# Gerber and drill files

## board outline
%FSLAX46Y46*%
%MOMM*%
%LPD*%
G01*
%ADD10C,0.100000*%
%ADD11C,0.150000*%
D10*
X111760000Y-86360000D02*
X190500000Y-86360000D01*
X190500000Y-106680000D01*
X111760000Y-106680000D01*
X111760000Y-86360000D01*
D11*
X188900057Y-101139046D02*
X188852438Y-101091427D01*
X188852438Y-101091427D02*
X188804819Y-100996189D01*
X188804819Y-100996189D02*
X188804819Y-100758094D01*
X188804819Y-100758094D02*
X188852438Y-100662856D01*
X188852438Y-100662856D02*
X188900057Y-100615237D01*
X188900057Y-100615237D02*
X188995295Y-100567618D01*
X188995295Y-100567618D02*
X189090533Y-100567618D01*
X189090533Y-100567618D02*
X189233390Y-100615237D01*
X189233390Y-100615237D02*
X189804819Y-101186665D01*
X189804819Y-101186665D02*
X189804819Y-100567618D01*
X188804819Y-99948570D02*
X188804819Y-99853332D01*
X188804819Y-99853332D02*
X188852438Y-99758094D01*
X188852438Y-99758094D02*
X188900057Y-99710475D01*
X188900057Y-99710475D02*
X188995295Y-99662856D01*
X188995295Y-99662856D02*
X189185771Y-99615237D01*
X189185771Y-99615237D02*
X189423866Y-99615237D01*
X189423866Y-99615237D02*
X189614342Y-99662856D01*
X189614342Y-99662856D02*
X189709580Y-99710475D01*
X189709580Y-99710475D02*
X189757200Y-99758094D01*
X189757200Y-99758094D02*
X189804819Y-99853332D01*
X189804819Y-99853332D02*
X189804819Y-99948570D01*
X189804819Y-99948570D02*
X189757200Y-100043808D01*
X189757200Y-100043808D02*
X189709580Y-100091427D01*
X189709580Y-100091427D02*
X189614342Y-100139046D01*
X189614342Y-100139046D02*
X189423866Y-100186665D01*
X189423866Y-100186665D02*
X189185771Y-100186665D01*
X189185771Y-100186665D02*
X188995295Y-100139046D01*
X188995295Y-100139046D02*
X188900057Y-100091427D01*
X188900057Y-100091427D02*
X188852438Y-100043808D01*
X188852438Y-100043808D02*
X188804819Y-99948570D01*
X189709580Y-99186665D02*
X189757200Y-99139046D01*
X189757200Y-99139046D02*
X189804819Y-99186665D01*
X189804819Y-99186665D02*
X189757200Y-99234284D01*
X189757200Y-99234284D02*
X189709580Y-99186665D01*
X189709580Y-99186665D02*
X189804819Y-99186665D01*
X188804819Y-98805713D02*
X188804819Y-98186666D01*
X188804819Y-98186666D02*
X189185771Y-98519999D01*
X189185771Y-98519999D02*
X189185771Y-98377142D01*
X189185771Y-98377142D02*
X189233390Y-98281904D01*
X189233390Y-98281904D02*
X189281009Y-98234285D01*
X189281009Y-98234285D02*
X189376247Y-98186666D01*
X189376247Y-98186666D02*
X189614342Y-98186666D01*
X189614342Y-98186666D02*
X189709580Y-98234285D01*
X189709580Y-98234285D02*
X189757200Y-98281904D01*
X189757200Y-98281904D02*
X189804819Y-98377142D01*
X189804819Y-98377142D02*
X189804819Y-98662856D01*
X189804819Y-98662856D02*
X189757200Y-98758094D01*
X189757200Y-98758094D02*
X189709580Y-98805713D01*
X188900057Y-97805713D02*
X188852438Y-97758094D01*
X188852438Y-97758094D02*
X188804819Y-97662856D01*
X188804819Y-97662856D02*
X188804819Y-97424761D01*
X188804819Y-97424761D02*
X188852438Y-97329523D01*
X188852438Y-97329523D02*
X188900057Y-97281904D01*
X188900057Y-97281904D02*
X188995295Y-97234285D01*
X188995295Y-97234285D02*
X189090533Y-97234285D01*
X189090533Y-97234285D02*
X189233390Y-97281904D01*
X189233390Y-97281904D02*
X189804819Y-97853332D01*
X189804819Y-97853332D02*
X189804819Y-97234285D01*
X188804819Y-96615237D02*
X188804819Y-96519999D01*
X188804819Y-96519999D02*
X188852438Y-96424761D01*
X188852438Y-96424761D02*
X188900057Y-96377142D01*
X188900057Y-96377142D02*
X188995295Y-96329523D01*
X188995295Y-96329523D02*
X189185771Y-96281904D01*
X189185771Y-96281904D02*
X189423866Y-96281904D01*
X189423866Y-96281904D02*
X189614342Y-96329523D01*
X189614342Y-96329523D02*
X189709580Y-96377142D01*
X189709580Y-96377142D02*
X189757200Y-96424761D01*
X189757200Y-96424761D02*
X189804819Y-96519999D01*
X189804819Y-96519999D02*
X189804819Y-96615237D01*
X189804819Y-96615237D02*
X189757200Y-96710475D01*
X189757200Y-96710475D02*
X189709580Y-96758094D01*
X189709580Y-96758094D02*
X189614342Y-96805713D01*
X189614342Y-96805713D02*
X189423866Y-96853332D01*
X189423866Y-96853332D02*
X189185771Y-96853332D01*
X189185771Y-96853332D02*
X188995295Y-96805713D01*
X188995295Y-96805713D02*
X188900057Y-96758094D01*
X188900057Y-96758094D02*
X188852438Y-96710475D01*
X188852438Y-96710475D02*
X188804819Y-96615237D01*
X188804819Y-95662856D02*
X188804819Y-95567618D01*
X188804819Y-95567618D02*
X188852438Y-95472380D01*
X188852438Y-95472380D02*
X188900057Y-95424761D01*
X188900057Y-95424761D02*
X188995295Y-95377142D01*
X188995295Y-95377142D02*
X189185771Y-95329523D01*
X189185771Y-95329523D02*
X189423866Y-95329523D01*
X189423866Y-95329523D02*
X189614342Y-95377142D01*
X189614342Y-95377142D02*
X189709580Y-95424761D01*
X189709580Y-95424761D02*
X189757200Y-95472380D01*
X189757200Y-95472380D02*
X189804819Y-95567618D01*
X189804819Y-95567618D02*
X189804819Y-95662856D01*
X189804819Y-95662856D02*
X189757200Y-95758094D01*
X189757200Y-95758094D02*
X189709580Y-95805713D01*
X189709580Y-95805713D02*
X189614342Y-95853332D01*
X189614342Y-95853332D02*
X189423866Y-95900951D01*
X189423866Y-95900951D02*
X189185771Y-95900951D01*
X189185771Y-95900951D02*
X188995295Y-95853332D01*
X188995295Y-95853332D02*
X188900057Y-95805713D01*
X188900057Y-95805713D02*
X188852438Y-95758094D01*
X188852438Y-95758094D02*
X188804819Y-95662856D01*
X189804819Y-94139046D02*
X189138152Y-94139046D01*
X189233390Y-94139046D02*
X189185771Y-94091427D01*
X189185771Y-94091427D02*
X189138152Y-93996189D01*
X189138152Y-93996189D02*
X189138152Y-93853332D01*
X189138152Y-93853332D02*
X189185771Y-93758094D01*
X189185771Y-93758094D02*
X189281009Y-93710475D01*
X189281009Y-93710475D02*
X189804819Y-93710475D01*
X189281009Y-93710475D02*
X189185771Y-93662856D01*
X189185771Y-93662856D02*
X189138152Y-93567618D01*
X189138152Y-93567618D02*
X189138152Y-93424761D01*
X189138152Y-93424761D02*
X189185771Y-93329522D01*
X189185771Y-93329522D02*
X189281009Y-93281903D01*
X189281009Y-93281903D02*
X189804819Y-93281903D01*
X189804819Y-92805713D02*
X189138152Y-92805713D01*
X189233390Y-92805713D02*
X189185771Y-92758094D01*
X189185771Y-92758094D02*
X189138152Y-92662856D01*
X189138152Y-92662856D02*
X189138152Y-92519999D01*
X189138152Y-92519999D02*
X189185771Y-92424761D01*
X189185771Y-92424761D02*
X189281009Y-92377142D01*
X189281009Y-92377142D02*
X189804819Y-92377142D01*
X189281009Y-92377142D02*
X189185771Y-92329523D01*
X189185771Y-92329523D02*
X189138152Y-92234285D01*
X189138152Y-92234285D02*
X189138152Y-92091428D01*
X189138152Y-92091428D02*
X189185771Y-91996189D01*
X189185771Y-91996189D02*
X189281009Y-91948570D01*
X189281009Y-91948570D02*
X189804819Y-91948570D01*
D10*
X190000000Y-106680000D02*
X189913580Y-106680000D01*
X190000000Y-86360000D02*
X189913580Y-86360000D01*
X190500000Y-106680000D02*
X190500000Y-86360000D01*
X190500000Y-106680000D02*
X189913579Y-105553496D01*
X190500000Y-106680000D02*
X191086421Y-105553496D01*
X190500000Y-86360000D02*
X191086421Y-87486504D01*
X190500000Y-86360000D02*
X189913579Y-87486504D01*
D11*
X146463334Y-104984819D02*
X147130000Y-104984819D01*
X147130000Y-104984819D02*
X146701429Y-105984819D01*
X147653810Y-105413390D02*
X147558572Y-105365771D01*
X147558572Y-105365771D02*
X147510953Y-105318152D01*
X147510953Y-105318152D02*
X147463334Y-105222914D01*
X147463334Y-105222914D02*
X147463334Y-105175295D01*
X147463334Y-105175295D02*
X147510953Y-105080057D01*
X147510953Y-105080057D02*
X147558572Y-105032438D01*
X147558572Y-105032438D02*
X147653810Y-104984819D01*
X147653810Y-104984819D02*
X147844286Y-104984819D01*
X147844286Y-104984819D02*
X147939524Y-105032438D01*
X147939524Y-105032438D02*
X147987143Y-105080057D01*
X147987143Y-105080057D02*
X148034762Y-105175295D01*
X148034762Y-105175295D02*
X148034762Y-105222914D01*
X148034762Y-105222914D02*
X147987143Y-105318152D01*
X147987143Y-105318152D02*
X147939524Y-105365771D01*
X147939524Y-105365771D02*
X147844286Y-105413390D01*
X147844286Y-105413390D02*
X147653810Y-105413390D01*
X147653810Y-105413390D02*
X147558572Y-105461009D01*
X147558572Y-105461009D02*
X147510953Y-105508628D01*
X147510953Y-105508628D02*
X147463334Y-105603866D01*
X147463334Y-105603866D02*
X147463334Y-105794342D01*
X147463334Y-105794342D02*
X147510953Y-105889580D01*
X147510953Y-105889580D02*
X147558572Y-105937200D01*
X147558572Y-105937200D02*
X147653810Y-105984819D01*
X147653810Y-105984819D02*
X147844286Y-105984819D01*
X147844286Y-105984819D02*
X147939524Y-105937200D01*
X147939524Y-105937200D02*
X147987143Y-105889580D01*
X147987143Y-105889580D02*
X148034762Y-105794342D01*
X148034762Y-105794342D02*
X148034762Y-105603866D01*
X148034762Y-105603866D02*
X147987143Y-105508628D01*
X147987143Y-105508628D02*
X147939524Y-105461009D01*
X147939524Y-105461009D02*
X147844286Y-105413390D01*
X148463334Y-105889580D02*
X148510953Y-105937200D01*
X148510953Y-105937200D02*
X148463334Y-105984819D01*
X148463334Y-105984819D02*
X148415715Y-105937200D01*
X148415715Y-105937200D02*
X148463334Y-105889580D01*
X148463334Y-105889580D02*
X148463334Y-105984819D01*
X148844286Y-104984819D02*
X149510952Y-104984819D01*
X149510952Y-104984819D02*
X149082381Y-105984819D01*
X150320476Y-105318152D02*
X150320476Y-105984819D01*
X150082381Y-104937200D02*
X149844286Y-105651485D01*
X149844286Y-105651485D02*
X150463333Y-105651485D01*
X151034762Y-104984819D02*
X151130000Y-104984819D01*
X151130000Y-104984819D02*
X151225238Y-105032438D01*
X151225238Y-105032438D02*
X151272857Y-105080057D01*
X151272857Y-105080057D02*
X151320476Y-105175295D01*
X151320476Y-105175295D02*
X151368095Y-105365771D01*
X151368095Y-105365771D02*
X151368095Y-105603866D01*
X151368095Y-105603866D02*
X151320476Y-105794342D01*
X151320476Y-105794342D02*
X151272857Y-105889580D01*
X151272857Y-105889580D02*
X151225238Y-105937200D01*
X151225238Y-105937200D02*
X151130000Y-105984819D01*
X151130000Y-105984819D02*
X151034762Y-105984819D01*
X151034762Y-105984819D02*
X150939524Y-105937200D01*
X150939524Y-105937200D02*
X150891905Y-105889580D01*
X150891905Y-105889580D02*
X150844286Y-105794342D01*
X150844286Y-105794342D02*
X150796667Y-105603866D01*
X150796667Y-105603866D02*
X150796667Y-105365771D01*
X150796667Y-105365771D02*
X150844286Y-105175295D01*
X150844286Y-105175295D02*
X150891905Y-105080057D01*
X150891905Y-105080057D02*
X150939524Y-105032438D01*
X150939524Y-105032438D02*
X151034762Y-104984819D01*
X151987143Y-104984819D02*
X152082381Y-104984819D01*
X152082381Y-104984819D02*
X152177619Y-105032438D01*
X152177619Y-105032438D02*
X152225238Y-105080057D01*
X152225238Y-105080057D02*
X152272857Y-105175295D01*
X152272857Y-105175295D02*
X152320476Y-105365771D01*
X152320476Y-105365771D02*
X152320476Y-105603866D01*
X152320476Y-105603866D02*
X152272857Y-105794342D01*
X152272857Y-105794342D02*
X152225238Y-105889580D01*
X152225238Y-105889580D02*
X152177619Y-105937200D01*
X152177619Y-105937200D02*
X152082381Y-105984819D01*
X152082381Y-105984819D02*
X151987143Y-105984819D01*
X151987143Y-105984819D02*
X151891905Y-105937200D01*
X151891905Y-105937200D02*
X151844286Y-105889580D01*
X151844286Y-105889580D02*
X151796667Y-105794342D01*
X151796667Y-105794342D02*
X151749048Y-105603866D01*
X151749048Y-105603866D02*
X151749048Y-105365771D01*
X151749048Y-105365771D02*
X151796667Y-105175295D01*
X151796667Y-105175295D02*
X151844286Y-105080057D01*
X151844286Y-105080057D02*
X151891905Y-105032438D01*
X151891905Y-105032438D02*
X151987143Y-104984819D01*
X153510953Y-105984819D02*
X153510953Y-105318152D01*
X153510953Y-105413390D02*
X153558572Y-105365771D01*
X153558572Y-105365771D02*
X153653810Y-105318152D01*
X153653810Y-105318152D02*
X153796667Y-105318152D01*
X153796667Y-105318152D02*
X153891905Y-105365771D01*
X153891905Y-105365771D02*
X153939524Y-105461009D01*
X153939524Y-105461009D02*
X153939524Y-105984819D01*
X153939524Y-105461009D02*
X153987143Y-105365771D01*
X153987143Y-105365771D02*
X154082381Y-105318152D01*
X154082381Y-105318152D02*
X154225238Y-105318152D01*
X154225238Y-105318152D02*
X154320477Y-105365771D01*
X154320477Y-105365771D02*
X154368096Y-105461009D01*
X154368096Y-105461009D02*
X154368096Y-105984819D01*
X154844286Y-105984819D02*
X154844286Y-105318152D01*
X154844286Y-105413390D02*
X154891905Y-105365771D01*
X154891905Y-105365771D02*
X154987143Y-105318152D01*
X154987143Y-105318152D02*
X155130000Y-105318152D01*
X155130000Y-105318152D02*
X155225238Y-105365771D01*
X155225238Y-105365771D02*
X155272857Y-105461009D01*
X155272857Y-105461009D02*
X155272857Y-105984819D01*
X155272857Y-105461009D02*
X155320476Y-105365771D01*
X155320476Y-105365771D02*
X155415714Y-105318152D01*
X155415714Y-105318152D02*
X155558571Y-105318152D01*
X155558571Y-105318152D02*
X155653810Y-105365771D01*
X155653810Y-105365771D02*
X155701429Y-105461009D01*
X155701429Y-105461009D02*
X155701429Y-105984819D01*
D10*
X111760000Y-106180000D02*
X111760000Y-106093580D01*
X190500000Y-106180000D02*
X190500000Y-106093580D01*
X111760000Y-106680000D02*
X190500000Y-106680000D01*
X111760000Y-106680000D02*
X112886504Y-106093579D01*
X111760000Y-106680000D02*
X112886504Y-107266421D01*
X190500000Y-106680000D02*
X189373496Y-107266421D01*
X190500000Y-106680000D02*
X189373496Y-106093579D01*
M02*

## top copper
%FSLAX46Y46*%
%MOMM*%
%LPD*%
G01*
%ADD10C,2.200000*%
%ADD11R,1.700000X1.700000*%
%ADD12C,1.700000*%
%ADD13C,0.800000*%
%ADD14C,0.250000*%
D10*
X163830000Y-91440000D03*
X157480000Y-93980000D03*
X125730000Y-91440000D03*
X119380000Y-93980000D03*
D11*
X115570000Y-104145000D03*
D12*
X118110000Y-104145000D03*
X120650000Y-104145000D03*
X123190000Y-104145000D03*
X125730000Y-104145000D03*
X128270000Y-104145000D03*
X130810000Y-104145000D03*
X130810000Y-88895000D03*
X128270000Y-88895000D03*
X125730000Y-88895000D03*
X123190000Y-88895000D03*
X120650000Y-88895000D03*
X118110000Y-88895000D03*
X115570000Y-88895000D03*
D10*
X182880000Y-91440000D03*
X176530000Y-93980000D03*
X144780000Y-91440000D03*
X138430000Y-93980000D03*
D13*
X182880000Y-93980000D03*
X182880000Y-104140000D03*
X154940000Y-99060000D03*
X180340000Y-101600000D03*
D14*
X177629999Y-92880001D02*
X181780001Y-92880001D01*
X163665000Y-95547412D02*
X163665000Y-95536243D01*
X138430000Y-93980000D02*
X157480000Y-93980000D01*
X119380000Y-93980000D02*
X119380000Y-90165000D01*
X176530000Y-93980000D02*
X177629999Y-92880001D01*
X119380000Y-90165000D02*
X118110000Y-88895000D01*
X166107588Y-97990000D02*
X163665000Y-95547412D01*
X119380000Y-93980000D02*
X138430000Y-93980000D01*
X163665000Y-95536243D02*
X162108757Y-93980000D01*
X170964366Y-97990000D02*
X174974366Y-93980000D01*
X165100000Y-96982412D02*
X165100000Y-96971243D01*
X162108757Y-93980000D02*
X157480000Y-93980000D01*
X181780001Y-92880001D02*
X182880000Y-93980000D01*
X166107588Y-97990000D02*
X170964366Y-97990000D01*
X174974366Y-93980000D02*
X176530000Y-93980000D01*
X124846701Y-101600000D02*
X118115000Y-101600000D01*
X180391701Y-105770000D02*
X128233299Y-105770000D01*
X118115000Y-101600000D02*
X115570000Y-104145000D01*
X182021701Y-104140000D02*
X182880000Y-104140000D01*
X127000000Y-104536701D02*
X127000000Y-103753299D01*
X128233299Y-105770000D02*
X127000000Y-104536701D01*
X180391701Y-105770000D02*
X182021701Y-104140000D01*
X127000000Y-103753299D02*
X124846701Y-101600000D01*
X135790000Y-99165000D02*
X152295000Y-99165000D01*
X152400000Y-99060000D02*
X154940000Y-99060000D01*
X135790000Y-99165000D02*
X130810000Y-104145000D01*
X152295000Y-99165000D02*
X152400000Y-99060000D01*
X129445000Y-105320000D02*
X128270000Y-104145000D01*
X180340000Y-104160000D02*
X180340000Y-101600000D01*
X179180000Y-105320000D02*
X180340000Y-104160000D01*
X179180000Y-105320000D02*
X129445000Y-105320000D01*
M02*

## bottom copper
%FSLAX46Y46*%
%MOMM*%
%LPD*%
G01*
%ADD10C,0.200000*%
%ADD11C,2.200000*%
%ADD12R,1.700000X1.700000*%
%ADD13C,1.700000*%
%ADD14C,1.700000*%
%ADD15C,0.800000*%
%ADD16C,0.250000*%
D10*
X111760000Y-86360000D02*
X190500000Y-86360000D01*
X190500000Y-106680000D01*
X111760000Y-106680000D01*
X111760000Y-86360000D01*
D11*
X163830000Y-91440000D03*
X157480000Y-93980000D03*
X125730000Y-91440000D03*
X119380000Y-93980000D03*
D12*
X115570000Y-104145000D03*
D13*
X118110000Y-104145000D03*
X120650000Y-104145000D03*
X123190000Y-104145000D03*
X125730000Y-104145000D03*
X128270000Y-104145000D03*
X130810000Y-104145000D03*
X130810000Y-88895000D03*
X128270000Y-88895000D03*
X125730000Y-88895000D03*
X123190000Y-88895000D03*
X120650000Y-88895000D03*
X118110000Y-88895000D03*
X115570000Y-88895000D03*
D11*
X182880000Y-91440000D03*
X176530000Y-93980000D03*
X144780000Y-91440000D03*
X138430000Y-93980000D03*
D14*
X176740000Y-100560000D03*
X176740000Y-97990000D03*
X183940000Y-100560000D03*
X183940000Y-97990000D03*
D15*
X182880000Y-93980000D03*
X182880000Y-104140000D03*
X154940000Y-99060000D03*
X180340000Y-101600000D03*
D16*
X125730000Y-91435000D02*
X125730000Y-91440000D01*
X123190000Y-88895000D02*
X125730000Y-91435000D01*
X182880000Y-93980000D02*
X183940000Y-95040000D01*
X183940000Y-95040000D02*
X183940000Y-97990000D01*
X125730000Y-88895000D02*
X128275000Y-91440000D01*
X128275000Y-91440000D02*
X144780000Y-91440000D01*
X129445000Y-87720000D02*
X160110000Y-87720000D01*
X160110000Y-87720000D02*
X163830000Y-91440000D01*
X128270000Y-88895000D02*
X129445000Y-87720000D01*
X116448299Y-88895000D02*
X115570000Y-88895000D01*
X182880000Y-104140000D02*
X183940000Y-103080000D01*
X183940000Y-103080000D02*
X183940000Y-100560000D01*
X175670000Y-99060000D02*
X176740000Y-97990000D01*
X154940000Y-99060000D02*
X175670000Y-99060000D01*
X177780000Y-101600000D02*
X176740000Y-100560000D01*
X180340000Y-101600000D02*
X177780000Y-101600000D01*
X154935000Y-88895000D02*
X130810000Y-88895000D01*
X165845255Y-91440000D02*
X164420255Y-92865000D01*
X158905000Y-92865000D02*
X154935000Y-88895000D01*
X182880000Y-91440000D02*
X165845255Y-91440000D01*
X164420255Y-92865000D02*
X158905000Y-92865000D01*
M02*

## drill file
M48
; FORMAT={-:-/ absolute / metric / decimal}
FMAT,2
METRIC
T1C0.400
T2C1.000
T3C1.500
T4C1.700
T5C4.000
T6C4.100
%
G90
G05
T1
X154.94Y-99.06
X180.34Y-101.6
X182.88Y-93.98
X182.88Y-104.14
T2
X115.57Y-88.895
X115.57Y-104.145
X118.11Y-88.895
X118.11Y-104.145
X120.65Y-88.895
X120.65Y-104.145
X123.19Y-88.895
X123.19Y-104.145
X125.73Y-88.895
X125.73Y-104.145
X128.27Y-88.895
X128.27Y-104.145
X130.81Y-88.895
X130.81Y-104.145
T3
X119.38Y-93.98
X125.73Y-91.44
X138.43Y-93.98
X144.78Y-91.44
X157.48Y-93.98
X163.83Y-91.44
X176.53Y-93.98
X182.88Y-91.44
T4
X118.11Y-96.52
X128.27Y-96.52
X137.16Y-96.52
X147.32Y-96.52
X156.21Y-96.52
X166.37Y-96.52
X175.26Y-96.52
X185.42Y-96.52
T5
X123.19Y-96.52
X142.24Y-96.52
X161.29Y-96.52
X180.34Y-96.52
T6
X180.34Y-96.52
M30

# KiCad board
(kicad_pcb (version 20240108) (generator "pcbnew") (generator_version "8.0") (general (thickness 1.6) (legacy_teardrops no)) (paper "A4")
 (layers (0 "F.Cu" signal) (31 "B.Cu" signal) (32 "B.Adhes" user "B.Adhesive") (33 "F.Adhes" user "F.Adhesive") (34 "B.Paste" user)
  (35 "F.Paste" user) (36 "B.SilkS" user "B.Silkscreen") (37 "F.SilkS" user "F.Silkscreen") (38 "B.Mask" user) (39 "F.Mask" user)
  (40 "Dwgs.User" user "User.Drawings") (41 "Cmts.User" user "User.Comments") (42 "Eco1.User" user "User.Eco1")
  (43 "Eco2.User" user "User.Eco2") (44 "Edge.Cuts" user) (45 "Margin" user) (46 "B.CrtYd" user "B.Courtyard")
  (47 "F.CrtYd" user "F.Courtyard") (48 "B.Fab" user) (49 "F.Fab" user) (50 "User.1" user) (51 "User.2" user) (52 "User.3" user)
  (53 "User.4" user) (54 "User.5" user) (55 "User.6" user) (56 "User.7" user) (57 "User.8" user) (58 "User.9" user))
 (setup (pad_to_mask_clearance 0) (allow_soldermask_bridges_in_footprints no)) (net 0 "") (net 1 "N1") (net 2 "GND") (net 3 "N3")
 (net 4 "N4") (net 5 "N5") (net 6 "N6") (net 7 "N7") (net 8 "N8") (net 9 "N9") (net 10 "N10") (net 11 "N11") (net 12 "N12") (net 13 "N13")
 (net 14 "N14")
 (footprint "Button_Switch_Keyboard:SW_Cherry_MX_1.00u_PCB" (layer "F.Cu") (at 163.83 91.44)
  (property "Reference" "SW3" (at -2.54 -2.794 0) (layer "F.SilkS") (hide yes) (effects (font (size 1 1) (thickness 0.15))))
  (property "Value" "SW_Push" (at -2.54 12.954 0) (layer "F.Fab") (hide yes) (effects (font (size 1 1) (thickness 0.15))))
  (pad "" np_thru_hole circle (at -7.62 5.08) (size 1.7 1.7) (drill 1.7) (layers "*.Cu" "*.Mask"))
  (pad "" np_thru_hole circle (at -2.54 5.08) (size 4 4) (drill 4) (layers "*.Cu" "*.Mask"))
  (pad "" np_thru_hole circle (at 2.54 5.08) (size 1.7 1.7) (drill 1.7) (layers "*.Cu" "*.Mask"))
  (pad "1" thru_hole circle (at 0 0) (size 2.2 2.2) (drill 1.5) (layers "*.Cu" "*.Mask") (remove_unused_layers no) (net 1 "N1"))
  (pad "2" thru_hole circle (at -6.35 2.54) (size 2.2 2.2) (drill 1.5) (layers "*.Cu" "*.Mask") (remove_unused_layers no) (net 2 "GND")))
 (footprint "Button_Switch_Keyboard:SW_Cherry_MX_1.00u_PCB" (layer "F.Cu") (at 125.73 91.44)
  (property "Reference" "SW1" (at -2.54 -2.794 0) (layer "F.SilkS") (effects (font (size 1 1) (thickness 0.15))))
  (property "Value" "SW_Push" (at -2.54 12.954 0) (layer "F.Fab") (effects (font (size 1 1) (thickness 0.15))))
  (pad "" np_thru_hole circle (at -7.62 5.08) (size 1.7 1.7) (drill 1.7) (layers "*.Cu" "*.Mask"))
  (pad "" np_thru_hole circle (at -2.54 5.08) (size 4 4) (drill 4) (layers "*.Cu" "*.Mask"))
  (pad "" np_thru_hole circle (at 2.54 5.08) (size 1.7 1.7) (drill 1.7) (layers "*.Cu" "*.Mask"))
  (pad "1" thru_hole circle (at 0 0) (size 2.2 2.2) (drill 1.5) (layers "*.Cu" "*.Mask") (remove_unused_layers no) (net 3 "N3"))
  (pad "2" thru_hole circle (at -6.35 2.54) (size 2.2 2.2) (drill 1.5) (layers "*.Cu" "*.Mask") (remove_unused_layers no) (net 2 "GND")))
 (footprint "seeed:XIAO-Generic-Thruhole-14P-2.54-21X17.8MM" (layer "F.Cu") (at 123.19 96.52 90)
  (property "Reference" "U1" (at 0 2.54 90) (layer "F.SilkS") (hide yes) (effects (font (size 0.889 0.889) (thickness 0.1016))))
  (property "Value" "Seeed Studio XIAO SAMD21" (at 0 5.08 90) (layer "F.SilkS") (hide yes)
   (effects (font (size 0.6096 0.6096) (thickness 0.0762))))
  (pad "1" thru_hole rect (at -7.625 -7.62 90) (size 1.7 1.7) (drill 1) (layers "*.Cu" "*.Mask") (remove_unused_layers no) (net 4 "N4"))
  (pad "2" thru_hole circle (at -7.625 -5.08 90) (size 1.7 1.7) (drill 1) (layers "*.Cu" "*.Mask") (remove_unused_layers no) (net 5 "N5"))
  (pad "3" thru_hole circle (at -7.625 -2.54 90) (size 1.7 1.7) (drill 1) (layers "*.Cu" "*.Mask") (remove_unused_layers no) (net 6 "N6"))
  (pad "4" thru_hole circle (at -7.625 0 90) (size 1.7 1.7) (drill 1) (layers "*.Cu" "*.Mask") (remove_unused_layers no) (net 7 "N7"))
  (pad "5" thru_hole circle (at -7.625 2.54 90) (size 1.7 1.7) (drill 1) (layers "*.Cu" "*.Mask") (remove_unused_layers no) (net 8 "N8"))
  (pad "6" thru_hole circle (at -7.625 5.08 270) (size 1.7 1.7) (drill 1) (layers "*.Cu" "*.Mask") (remove_unused_layers no) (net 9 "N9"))
  (pad "7" thru_hole circle (at -7.625 7.62 90) (size 1.7 1.7) (drill 1) (layers "*.Cu" "*.Mask") (remove_unused_layers no) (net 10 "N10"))
  (pad "8" thru_hole circle (at 7.625 7.62 90) (size 1.7 1.7) (drill 1) (layers "*.Cu" "*.Mask") (remove_unused_layers no) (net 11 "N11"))
  (pad "9" thru_hole circle (at 7.625 5.08 90) (size 1.7 1.7) (drill 1) (layers "*.Cu" "*.Mask") (remove_unused_layers no) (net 1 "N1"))
  (pad "10" thru_hole circle (at 7.625 2.54 90) (size 1.7 1.7) (drill 1) (layers "*.Cu" "*.Mask") (remove_unused_layers no) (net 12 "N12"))
  (pad "11" thru_hole circle (at 7.625 0 90) (size 1.7 1.7) (drill 1) (layers "*.Cu" "*.Mask") (remove_unused_layers no) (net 3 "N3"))
  (pad "12" thru_hole circle (at 7.625 -2.54 90) (size 1.7 1.7) (drill 1) (layers "*.Cu" "*.Mask") (remove_unused_layers no) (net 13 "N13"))
  (pad "13" thru_hole circle (at 7.625 -5.08 90) (size 1.7 1.7) (drill 1) (layers "*.Cu" "*.Mask") (remove_unused_layers no) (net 2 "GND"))
  (pad "14" thru_hole circle (at 7.625 -7.62 90) (size 1.7 1.7) (drill 1) (layers "*.Cu" "*.Mask") (remove_unused_layers no) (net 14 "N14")))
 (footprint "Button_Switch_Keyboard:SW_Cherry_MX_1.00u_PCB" (layer "F.Cu") (at 182.88 91.44)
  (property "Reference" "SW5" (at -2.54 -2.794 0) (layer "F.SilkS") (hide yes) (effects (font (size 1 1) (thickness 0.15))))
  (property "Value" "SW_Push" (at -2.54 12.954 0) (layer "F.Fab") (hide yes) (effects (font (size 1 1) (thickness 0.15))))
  (pad "" np_thru_hole circle (at -7.62 5.08) (size 1.7 1.7) (drill 1.7) (layers "*.Cu" "*.Mask"))
  (pad "" np_thru_hole circle (at -2.54 5.08) (size 4 4) (drill 4) (layers "*.Cu" "*.Mask"))
  (pad "" np_thru_hole circle (at 2.54 5.08) (size 1.7 1.7) (drill 1.7) (layers "*.Cu" "*.Mask"))
  (pad "1" thru_hole circle (at 0 0) (size 2.2 2.2) (drill 1.5) (layers "*.Cu" "*.Mask") (remove_unused_layers no) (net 11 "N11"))
  (pad "2" thru_hole circle (at -6.35 2.54) (size 2.2 2.2) (drill 1.5) (layers "*.Cu" "*.Mask") (remove_unused_layers no) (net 2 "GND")))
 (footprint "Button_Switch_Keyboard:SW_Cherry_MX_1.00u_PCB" (layer "F.Cu") (at 144.78 91.44)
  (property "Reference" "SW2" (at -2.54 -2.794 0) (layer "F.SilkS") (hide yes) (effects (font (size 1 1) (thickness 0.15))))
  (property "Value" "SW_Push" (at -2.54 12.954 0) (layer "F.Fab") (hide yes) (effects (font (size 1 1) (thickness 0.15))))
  (pad "" np_thru_hole circle (at -7.62 5.08) (size 1.7 1.7) (drill 1.7) (layers "*.Cu" "*.Mask"))
  (pad "" np_thru_hole circle (at -2.54 5.08) (size 4 4) (drill 4) (layers "*.Cu" "*.Mask"))
  (pad "" np_thru_hole circle (at 2.54 5.08) (size 1.7 1.7) (drill 1.7) (layers "*.Cu" "*.Mask"))
  (pad "1" thru_hole circle (at 0 0) (size 2.2 2.2) (drill 1.5) (layers "*.Cu" "*.Mask") (remove_unused_layers no) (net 12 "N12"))
  (pad "2" thru_hole circle (at -6.35 2.54) (size 2.2 2.2) (drill 1.5) (layers "*.Cu" "*.Mask") (remove_unused_layers no) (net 2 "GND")))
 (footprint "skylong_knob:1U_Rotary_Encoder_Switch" (layer "B.Cu") (at 180.34 96.52 180)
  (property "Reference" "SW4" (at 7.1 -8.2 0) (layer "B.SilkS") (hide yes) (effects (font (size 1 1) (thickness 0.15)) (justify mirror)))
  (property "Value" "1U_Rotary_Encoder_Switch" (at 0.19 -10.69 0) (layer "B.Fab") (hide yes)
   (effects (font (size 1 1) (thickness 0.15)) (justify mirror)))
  (pad "" np_thru_hole circle (at 0 0 180) (size 4.1 4.1) (drill 4.1) (layers "F&B.Cu" "*.Mask"))
  (pad "1" smd circle (at 3.6 -4.04 180) (size 1.7 1.7) (layers "B.Cu" "B.Paste" "B.Mask") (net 9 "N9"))
  (pad "2" smd circle (at 3.6 -1.47 180) (size 1.7 1.7) (layers "B.Cu" "B.Paste" "B.Mask") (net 10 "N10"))
  (pad "3" smd circle (at -3.6 -4.04 180) (size 1.7 1.7) (layers "B.Cu" "B.Paste" "B.Mask") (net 4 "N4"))
  (pad "4" smd circle (at -3.6 -1.47 180) (size 1.7 1.7) (layers "B.Cu" "B.Paste" "B.Mask") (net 2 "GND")))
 (gr_rect (start 111.76 86.36) (end 190.5 106.68) (stroke (width 0.2) (type default)) (fill none) (layer "B.Cu"))
 (gr_rect (start 111.76 86.36) (end 190.5 106.68) (stroke (width 0.1) (type default)) (fill none) (layer "Edge.Cuts"))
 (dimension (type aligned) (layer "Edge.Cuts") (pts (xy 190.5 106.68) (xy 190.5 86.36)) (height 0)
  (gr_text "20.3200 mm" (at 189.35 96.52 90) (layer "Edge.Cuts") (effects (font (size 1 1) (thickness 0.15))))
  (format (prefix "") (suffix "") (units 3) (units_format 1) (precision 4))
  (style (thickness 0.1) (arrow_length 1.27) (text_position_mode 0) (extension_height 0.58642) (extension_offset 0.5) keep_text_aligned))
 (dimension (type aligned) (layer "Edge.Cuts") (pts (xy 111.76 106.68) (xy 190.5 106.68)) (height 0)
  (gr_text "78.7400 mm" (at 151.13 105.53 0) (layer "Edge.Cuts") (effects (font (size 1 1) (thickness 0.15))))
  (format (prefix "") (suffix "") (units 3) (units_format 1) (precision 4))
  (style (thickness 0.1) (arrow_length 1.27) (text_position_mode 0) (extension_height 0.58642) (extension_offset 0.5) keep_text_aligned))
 (segment (start 125.73 91.435) (end 125.73 91.44) (width 0.25) (layer "B.Cu") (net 3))
 (segment (start 123.19 88.895) (end 125.73 91.435) (width 0.25) (layer "B.Cu") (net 3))
 (segment (start 177.629999 92.880001) (end 181.780001 92.880001) (width 0.25) (layer "F.Cu") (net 2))
 (segment (start 163.665 95.547412) (end 163.665 95.536243) (width 0.25) (layer "F.Cu") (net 2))
 (segment (start 138.43 93.98) (end 157.48 93.98) (width 0.25) (layer "F.Cu") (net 2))
 (segment (start 119.38 93.98) (end 119.38 90.165) (width 0.25) (layer "F.Cu") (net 2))
 (segment (start 176.53 93.98) (end 177.629999 92.880001) (width 0.25) (layer "F.Cu") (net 2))
 (segment (start 119.38 90.165) (end 118.11 88.895) (width 0.25) (layer "F.Cu") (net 2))
 (segment (start 166.107588 97.99) (end 163.665 95.547412) (width 0.25) (layer "F.Cu") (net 2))
 (segment (start 119.38 93.98) (end 138.43 93.98) (width 0.25) (layer "F.Cu") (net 2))
 (segment (start 163.665 95.536243) (end 162.108757 93.98) (width 0.25) (layer "F.Cu") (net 2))
 (segment (start 170.964366 97.99) (end 174.974366 93.98) (width 0.25) (layer "F.Cu") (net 2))
 (segment (start 165.1 96.982412) (end 165.1 96.971243) (width 0.25) (layer "F.Cu") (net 2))
 (segment (start 162.108757 93.98) (end 157.48 93.98) (width 0.25) (layer "F.Cu") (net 2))
 (segment (start 181.780001 92.880001) (end 182.88 93.98) (width 0.25) (layer "F.Cu") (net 2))
 (segment (start 166.107588 97.99) (end 170.964366 97.99) (width 0.25) (layer "F.Cu") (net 2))
 (segment (start 174.974366 93.98) (end 176.53 93.98) (width 0.25) (layer "F.Cu") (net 2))
 (via (at 182.88 93.98) (size 0.8) (drill 0.4) (layers "F.Cu" "B.Cu") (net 2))
 (segment (start 182.88 93.98) (end 183.94 95.04) (width 0.25) (layer "B.Cu") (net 2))
 (segment (start 183.94 95.04) (end 183.94 97.99) (width 0.25) (layer "B.Cu") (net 2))
 (segment (start 125.73 88.895) (end 128.275 91.44) (width 0.25) (layer "B.Cu") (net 12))
 (segment (start 128.275 91.44) (end 144.78 91.44) (width 0.25) (layer "B.Cu") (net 12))
 (segment (start 129.445 87.72) (end 160.11 87.72) (width 0.25) (layer "B.Cu") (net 1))
 (segment (start 160.11 87.72) (end 163.83 91.44) (width 0.25) (layer "B.Cu") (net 1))
 (segment (start 128.27 88.895) (end 129.445 87.72) (width 0.25) (layer "B.Cu") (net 1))
 (segment (start 116.448299 88.895) (end 115.57 88.895) (width 0.25) (layer "B.Cu") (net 14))
 (segment (start 124.846701 101.6) (end 118.115 101.6) (width 0.25) (layer "F.Cu") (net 4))
 (segment (start 180.391701 105.77) (end 128.233299 105.77) (width 0.25) (layer "F.Cu") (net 4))
 (segment (start 118.115 101.6) (end 115.57 104.145) (width 0.25) (layer "F.Cu") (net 4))
 (segment (start 182.021701 104.14) (end 182.88 104.14) (width 0.25) (layer "F.Cu") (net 4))
 (segment (start 127 104.536701) (end 127 103.753299) (width 0.25) (layer "F.Cu") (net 4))
 (segment (start 128.233299 105.77) (end 127 104.536701) (width 0.25) (layer "F.Cu") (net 4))
 (segment (start 180.391701 105.77) (end 182.021701 104.14) (width 0.25) (layer "F.Cu") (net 4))
 (segment (start 127 103.753299) (end 124.846701 101.6) (width 0.25) (layer "F.Cu") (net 4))
 (via (at 182.88 104.14) (size 0.8) (drill 0.4) (layers "F.Cu" "B.Cu") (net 4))
 (segment (start 182.88 104.14) (end 183.94 103.08) (width 0.25) (layer "B.Cu") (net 4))
 (segment (start 183.94 103.08) (end 183.94 100.56) (width 0.25) (layer "B.Cu") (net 4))
 (segment (start 135.79 99.165) (end 152.295 99.165) (width 0.25) (layer "F.Cu") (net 10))
 (segment (start 152.4 99.06) (end 154.94 99.06) (width 0.25) (layer "F.Cu") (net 10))
 (segment (start 135.79 99.165) (end 130.81 104.145) (width 0.25) (layer "F.Cu") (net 10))
 (segment (start 152.295 99.165) (end 152.4 99.06) (width 0.25) (layer "F.Cu") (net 10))
 (via (at 154.94 99.06) (size 0.8) (drill 0.4) (layers "F.Cu" "B.Cu") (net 10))
 (segment (start 175.67 99.06) (end 176.74 97.99) (width 0.25) (layer "B.Cu") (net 10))
 (segment (start 154.94 99.06) (end 175.67 99.06) (width 0.25) (layer "B.Cu") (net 10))
 (segment (start 129.445 105.32) (end 128.27 104.145) (width 0.25) (layer "F.Cu") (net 9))
 (segment (start 180.34 104.16) (end 180.34 101.6) (width 0.25) (layer "F.Cu") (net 9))
 (segment (start 179.18 105.32) (end 180.34 104.16) (width 0.25) (layer "F.Cu") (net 9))
 (segment (start 179.18 105.32) (end 129.445 105.32) (width 0.25) (layer "F.Cu") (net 9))
 (via (at 180.34 101.6) (size 0.8) (drill 0.4) (layers "F.Cu" "B.Cu") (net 9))
 (segment (start 177.78 101.6) (end 176.74 100.56) (width 0.25) (layer "B.Cu") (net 9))
 (segment (start 180.34 101.6) (end 177.78 101.6) (width 0.25) (layer "B.Cu") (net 9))
 (segment (start 154.935 88.895) (end 130.81 88.895) (width 0.25) (layer "B.Cu") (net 11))
 (segment (start 165.845255 91.44) (end 164.420255 92.865) (width 0.25) (layer "B.Cu") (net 11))
 (segment (start 158.905 92.865) (end 154.935 88.895) (width 0.25) (layer "B.Cu") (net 11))
 (segment (start 182.88 91.44) (end 165.845255 91.44) (width 0.25) (layer "B.Cu") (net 11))
 (segment (start 164.420255 92.865) (end 158.905 92.865) (width 0.25) (layer "B.Cu") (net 11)))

